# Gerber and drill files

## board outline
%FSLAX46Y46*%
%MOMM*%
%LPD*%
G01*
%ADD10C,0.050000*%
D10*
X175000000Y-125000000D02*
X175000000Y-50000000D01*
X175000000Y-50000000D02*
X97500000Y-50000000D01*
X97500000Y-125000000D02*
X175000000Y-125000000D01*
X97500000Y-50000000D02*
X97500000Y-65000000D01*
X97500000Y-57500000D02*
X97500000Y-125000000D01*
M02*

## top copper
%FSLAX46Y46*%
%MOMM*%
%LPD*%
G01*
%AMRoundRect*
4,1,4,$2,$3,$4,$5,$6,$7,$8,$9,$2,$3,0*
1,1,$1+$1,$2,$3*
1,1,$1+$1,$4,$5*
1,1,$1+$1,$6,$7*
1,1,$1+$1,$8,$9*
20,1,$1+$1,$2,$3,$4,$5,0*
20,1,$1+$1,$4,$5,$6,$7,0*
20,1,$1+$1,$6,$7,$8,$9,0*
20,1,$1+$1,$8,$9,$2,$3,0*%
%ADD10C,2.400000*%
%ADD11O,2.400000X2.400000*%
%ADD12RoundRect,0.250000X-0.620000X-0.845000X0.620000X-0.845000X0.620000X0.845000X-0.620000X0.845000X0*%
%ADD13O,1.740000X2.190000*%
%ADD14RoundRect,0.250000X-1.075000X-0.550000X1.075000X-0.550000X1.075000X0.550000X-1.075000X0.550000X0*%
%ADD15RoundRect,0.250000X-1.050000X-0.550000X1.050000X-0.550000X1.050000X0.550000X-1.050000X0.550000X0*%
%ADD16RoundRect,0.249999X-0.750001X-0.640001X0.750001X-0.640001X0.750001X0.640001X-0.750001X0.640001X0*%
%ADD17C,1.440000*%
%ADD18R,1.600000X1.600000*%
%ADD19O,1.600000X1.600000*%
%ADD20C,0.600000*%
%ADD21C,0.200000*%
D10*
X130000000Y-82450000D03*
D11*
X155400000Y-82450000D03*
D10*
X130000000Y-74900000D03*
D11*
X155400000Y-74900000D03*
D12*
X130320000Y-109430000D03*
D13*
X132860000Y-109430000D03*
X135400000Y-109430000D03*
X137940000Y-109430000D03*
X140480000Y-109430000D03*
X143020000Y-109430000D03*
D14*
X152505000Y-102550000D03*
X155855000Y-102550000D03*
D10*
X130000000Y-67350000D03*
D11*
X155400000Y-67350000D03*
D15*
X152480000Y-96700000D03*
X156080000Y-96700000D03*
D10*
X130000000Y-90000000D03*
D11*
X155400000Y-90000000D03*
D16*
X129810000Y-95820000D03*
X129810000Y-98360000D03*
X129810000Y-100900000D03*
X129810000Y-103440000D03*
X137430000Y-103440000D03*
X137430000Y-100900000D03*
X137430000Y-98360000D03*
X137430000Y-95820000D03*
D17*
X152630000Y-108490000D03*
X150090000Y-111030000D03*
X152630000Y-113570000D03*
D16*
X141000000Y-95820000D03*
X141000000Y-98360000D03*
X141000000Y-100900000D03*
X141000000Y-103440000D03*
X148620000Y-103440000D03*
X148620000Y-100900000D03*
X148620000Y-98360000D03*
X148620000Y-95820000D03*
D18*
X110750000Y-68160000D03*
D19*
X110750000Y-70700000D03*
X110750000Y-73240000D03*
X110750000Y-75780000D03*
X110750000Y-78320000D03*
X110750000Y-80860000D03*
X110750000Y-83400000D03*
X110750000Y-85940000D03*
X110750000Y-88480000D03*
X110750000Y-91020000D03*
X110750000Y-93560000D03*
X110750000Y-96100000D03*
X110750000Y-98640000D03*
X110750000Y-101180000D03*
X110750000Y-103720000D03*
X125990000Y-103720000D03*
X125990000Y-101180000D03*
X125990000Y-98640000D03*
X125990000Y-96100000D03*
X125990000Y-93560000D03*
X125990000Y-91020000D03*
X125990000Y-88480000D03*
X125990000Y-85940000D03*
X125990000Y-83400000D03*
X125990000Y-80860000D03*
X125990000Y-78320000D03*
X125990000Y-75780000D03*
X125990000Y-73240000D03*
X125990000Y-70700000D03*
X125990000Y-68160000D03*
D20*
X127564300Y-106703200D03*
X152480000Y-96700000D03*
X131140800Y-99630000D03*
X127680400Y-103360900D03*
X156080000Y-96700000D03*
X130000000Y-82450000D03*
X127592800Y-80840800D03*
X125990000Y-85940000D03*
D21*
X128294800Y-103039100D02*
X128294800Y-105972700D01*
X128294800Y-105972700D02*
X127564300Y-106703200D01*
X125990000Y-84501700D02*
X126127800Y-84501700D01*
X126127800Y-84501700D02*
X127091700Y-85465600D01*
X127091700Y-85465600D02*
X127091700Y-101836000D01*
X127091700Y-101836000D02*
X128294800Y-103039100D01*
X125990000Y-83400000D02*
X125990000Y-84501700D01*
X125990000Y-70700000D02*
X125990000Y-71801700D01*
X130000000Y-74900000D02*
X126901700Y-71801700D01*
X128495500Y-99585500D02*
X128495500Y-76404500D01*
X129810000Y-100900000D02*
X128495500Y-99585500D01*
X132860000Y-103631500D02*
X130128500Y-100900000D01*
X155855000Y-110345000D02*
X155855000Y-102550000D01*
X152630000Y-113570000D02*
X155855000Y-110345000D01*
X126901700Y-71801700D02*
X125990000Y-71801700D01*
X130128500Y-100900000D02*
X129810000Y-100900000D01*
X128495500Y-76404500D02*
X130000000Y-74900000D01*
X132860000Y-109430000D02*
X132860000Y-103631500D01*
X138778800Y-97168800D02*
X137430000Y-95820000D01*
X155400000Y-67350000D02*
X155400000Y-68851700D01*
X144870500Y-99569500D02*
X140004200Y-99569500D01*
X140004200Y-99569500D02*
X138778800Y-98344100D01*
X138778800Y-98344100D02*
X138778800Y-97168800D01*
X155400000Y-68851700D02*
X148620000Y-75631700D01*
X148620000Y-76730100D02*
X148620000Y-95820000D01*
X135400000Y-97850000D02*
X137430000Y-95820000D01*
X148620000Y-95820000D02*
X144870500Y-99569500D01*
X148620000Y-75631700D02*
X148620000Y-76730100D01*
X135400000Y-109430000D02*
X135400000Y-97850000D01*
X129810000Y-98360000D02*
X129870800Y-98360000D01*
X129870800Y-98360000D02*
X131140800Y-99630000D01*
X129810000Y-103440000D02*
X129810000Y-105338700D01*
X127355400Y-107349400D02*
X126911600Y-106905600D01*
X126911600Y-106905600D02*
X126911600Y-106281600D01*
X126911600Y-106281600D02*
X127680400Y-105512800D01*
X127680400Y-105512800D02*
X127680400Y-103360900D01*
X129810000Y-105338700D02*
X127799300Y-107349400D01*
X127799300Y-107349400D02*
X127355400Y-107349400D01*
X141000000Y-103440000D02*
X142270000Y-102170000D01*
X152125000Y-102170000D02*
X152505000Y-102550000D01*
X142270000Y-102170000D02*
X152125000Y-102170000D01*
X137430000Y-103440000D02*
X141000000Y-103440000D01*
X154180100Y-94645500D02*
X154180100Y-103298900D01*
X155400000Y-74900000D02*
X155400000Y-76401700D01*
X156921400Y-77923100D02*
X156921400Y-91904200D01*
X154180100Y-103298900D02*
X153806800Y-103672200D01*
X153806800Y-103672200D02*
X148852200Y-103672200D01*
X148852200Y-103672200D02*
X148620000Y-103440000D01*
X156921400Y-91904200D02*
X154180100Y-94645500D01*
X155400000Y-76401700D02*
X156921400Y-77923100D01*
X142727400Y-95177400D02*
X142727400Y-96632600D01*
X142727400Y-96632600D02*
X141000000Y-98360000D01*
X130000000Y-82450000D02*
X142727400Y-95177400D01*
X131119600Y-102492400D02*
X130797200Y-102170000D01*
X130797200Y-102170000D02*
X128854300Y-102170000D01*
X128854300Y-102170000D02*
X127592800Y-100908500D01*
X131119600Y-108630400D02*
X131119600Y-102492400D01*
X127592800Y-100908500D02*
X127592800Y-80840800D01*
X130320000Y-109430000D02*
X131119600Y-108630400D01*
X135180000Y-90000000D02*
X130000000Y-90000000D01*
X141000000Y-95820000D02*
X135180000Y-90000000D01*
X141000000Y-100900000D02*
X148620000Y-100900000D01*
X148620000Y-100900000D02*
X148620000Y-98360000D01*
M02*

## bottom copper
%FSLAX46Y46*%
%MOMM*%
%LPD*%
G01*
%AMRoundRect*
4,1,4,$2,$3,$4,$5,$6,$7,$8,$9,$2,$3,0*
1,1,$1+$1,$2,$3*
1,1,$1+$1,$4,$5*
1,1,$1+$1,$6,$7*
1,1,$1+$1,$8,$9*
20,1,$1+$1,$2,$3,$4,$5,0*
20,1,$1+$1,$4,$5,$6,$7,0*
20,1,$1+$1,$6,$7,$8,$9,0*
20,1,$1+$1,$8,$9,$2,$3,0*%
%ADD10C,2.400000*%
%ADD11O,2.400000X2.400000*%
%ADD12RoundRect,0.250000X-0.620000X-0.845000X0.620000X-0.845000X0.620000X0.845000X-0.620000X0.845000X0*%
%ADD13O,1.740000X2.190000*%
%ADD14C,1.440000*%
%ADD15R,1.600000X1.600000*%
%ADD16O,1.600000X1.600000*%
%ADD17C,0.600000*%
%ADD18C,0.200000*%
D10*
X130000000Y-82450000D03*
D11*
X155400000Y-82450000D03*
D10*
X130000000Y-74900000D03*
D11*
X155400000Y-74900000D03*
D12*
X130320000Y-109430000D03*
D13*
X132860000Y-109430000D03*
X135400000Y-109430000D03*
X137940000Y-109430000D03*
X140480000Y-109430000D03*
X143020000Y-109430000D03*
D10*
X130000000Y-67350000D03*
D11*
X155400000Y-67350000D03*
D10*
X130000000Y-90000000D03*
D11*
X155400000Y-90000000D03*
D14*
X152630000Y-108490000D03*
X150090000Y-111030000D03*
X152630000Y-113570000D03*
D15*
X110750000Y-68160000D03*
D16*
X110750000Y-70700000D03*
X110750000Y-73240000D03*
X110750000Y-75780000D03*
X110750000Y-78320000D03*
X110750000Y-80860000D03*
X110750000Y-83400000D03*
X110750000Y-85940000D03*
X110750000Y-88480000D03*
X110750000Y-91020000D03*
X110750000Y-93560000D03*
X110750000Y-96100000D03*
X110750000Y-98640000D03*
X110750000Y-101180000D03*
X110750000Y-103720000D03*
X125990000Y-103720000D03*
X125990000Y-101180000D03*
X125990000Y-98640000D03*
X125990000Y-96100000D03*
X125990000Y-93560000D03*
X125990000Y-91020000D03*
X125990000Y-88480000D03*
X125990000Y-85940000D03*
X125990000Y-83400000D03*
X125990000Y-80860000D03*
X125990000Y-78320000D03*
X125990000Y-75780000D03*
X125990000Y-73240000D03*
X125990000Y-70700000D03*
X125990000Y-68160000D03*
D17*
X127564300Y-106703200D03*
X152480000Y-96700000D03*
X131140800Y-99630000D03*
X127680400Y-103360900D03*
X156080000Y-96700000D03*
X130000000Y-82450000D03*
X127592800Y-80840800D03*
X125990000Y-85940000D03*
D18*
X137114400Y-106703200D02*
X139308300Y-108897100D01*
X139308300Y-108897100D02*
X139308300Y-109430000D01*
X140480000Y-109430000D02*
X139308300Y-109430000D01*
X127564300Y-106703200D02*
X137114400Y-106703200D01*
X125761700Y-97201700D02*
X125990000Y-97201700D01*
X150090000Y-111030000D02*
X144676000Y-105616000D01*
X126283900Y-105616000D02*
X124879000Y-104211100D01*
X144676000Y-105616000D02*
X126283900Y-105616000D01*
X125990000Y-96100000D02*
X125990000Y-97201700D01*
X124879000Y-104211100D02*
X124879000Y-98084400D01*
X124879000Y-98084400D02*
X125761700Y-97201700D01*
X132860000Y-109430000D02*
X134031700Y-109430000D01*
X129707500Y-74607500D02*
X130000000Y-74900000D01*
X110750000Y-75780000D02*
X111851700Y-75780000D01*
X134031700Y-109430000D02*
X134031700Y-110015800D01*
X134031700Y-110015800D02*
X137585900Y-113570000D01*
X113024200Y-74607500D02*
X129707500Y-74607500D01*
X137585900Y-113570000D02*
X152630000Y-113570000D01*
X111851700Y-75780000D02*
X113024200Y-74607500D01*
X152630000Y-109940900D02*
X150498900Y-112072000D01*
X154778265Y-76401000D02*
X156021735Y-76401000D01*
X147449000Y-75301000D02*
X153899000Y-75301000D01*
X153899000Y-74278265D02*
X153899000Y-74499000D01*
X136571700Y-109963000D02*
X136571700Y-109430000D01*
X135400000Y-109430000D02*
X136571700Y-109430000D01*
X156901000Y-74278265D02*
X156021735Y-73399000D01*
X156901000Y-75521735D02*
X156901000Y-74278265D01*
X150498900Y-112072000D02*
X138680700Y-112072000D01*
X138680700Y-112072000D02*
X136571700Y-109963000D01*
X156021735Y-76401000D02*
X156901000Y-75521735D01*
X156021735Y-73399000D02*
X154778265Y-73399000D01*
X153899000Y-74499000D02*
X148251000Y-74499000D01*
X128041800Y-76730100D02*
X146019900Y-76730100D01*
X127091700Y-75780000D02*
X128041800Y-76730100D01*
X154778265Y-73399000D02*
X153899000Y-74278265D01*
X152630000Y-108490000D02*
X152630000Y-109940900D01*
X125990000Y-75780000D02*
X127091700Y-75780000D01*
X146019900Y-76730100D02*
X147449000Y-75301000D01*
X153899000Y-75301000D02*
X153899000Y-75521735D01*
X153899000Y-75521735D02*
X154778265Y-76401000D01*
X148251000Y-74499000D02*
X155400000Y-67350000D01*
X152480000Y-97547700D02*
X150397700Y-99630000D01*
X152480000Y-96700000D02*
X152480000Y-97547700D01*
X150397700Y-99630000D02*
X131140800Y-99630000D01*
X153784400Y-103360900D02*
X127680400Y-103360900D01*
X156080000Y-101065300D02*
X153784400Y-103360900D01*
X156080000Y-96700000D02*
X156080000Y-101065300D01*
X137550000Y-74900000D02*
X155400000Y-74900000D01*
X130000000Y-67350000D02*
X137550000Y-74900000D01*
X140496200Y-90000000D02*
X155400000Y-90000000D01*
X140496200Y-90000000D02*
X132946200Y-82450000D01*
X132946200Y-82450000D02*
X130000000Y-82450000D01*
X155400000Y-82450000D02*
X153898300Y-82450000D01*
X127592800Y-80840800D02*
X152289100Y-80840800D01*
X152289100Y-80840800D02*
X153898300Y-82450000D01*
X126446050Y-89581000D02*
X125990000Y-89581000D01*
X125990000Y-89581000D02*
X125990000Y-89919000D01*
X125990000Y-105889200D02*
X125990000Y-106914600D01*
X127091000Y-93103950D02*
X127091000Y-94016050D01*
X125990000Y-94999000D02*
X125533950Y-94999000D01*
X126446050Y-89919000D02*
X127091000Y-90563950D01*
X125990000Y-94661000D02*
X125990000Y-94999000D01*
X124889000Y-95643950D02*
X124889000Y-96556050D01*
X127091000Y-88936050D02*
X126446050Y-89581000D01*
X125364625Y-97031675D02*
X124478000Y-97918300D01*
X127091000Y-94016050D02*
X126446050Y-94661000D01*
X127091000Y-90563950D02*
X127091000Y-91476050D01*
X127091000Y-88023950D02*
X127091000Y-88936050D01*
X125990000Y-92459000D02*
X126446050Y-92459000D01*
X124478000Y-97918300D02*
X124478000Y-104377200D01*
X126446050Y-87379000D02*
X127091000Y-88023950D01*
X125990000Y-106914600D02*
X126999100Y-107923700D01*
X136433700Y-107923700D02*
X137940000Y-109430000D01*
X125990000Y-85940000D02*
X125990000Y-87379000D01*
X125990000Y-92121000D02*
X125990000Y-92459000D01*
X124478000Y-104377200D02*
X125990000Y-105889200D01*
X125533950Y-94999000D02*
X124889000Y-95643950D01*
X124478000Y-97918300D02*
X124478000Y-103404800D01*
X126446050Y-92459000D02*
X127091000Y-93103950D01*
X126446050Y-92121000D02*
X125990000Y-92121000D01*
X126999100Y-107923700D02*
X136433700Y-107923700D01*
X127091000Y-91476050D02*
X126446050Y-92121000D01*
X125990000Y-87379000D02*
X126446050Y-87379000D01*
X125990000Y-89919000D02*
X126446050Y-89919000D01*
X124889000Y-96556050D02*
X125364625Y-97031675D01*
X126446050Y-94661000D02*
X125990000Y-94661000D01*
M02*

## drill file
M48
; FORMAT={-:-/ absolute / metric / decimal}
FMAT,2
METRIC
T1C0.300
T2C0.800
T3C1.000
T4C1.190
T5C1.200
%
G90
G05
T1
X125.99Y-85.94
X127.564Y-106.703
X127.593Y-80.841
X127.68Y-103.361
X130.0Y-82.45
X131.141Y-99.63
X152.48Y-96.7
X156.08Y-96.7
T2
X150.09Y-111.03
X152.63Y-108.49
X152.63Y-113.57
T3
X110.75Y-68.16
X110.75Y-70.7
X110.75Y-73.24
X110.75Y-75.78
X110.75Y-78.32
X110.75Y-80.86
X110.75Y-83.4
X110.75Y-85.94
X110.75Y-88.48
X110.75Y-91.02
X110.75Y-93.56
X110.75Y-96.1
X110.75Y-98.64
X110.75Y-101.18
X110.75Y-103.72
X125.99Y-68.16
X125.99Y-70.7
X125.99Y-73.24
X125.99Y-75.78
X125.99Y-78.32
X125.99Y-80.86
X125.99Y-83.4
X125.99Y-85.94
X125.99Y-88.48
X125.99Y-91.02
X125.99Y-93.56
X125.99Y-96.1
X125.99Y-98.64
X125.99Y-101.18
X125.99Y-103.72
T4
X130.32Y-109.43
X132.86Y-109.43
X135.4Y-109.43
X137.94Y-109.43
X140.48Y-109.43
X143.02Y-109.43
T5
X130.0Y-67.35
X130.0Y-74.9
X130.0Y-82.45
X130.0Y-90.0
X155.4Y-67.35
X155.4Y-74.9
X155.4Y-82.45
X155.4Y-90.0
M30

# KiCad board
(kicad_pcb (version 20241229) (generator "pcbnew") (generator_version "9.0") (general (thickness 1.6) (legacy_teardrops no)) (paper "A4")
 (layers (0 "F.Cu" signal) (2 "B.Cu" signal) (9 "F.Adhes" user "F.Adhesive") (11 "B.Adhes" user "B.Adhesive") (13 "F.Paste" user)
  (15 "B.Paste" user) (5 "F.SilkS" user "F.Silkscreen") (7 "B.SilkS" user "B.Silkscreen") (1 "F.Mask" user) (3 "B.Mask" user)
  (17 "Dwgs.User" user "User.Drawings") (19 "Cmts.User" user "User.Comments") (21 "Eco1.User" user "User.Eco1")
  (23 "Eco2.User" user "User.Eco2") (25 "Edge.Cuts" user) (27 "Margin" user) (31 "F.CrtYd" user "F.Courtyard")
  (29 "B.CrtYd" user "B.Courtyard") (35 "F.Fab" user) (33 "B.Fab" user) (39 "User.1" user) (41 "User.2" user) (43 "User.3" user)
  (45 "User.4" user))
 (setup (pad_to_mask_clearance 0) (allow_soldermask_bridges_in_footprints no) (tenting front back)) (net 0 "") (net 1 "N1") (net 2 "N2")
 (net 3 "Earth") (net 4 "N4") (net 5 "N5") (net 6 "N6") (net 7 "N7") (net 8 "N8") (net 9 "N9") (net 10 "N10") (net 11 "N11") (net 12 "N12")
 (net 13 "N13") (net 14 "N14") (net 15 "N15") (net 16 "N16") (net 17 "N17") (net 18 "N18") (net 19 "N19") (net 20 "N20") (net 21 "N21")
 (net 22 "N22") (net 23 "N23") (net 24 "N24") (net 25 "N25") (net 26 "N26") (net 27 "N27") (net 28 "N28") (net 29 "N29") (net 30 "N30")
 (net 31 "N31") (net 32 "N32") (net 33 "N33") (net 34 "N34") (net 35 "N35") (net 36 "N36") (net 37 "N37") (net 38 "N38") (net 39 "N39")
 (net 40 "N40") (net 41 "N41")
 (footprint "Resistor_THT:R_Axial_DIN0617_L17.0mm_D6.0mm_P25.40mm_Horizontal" (layer "F.Cu") (at 130 82.45)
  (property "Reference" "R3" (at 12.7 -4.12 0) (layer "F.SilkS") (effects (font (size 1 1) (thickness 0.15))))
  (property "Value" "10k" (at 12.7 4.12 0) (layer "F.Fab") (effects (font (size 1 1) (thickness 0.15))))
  (pad "1" thru_hole circle (at 0 0) (size 2.4 2.4) (drill 1.2) (layers "*.Cu" "*.Mask") (remove_unused_layers no) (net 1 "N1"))
  (pad "2" thru_hole oval (at 25.4 0) (size 2.4 2.4) (drill 1.2) (layers "*.Cu" "*.Mask") (remove_unused_layers no) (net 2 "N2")))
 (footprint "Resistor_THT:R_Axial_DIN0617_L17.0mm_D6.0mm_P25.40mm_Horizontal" (layer "F.Cu") (at 130 74.9)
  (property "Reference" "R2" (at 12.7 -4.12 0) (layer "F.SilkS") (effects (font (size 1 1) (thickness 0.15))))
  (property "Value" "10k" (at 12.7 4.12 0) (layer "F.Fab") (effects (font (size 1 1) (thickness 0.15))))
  (pad "1" thru_hole circle (at 0 0) (size 2.4 2.4) (drill 1.2) (layers "*.Cu" "*.Mask") (remove_unused_layers no) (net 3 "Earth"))
  (pad "2" thru_hole oval (at 25.4 0) (size 2.4 2.4) (drill 1.2) (layers "*.Cu" "*.Mask") (remove_unused_layers no) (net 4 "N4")))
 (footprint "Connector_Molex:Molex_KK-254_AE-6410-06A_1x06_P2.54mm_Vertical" (layer "F.Cu") (at 130.32 109.43)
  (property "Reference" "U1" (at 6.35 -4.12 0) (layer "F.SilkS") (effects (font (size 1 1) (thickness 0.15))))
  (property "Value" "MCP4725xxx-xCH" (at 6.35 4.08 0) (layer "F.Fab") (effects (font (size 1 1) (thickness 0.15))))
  (pad "1" thru_hole roundrect (at 0 0) (size 1.74 2.19) (drill 1.19) (layers "*.Cu" "*.Mask") (remove_unused_layers no)
   (roundrect_rratio 0.143678) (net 2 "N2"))
  (pad "2" thru_hole oval (at 2.54 0) (size 1.74 2.19) (drill 1.19) (layers "*.Cu" "*.Mask") (remove_unused_layers no) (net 3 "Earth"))
  (pad "3" thru_hole oval (at 5.08 0) (size 1.74 2.19) (drill 1.19) (layers "*.Cu" "*.Mask") (remove_unused_layers no) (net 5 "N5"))
  (pad "4" thru_hole oval (at 7.62 0) (size 1.74 2.19) (drill 1.19) (layers "*.Cu" "*.Mask") (remove_unused_layers no) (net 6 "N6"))
  (pad "5" thru_hole oval (at 10.16 0) (size 1.74 2.19) (drill 1.19) (layers "*.Cu" "*.Mask") (remove_unused_layers no) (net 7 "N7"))
  (pad "6" thru_hole oval (at 12.7 0) (size 1.74 2.19) (drill 1.19) (layers "*.Cu" "*.Mask") (remove_unused_layers no) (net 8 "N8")))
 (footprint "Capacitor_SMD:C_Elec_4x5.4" (layer "F.Cu") (at 154.18 102.55)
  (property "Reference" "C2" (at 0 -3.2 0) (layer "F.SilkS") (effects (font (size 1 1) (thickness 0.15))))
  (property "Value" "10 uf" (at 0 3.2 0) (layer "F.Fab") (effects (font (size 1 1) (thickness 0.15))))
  (pad "1" smd roundrect (at -1.675 0) (size 2.65 1.6) (layers "F.Cu" "F.Mask" "F.Paste") (roundrect_rratio 0.15625) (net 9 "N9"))
  (pad "2" smd roundrect (at 1.675 0) (size 2.65 1.6) (layers "F.Cu" "F.Mask" "F.Paste") (roundrect_rratio 0.15625) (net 3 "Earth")))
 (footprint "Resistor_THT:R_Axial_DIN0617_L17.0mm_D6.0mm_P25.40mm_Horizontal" (layer "F.Cu") (at 130 67.35)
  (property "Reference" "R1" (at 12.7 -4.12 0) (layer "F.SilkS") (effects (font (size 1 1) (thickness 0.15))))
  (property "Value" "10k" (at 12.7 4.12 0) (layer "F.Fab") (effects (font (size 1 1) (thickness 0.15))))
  (pad "1" thru_hole circle (at 0 0) (size 2.4 2.4) (drill 1.2) (layers "*.Cu" "*.Mask") (remove_unused_layers no) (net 4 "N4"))
  (pad "2" thru_hole oval (at 25.4 0) (size 2.4 2.4) (drill 1.2) (layers "*.Cu" "*.Mask") (remove_unused_layers no) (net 5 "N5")))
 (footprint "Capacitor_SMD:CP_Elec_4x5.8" (layer "F.Cu") (at 154.28 96.7)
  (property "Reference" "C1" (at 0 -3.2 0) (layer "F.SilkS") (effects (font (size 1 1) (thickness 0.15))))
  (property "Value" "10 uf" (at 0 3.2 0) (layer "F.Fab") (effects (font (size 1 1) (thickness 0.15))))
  (pad "1" smd roundrect (at -1.8 0) (size 2.6 1.6) (layers "F.Cu" "F.Mask" "F.Paste") (roundrect_rratio 0.15625) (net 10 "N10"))
  (pad "2" smd roundrect (at 1.8 0) (size 2.6 1.6) (layers "F.Cu" "F.Mask" "F.Paste") (roundrect_rratio 0.15625) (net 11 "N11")))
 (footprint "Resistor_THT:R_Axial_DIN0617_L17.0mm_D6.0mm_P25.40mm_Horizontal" (layer "F.Cu") (at 130 90)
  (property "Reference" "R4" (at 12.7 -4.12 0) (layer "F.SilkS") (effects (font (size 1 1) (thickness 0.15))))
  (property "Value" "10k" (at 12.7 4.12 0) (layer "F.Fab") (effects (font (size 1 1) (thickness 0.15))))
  (pad "1" thru_hole circle (at 0 0) (size 2.4 2.4) (drill 1.2) (layers "*.Cu" "*.Mask") (remove_unused_layers no) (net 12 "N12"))
  (pad "2" thru_hole oval (at 25.4 0) (size 2.4 2.4) (drill 1.2) (layers "*.Cu" "*.Mask") (remove_unused_layers no) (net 1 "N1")))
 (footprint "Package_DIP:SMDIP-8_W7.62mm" (layer "F.Cu") (at 133.62 99.63)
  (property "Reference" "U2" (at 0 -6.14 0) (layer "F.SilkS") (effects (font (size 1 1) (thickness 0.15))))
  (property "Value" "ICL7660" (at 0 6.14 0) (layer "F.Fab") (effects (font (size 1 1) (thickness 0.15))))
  (pad "1" smd roundrect (at -3.81 -3.81) (size 2 1.78) (layers "F.Cu" "F.Mask" "F.Paste") (roundrect_rratio 0.140449) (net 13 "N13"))
  (pad "2" smd roundrect (at -3.81 -1.27) (size 2 1.78) (layers "F.Cu" "F.Mask" "F.Paste") (roundrect_rratio 0.140449) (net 10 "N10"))
  (pad "3" smd roundrect (at -3.81 1.27) (size 2 1.78) (layers "F.Cu" "F.Mask" "F.Paste") (roundrect_rratio 0.140449) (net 3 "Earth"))
  (pad "4" smd roundrect (at -3.81 3.81) (size 2 1.78) (layers "F.Cu" "F.Mask" "F.Paste") (roundrect_rratio 0.140449) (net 11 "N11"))
  (pad "5" smd roundrect (at 3.81 3.81) (size 2 1.78) (layers "F.Cu" "F.Mask" "F.Paste") (roundrect_rratio 0.140449) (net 9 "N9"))
  (pad "6" smd roundrect (at 3.81 1.27) (size 2 1.78) (layers "F.Cu" "F.Mask" "F.Paste") (roundrect_rratio 0.140449) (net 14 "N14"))
  (pad "7" smd roundrect (at 3.81 -1.27) (size 2 1.78) (layers "F.Cu" "F.Mask" "F.Paste") (roundrect_rratio 0.140449) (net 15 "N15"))
  (pad "8" smd roundrect (at 3.81 -3.81) (size 2 1.78) (layers "F.Cu" "F.Mask" "F.Paste") (roundrect_rratio 0.140449) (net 5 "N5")))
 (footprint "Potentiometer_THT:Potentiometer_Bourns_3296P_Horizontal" (layer "F.Cu") (at 152.63 108.49)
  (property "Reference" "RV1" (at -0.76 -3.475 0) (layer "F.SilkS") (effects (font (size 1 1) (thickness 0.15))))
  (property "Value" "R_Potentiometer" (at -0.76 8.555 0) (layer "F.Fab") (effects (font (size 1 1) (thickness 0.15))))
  (pad "1" thru_hole circle (at 0 0) (size 1.44 1.44) (drill 0.8) (layers "*.Cu" "*.Mask") (remove_unused_layers no) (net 5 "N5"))
  (pad "2" thru_hole circle (at -2.54 2.54) (size 1.44 1.44) (drill 0.8) (layers "*.Cu" "*.Mask") (remove_unused_layers no) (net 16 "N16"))
  (pad "3" thru_hole circle (at 0 5.08) (size 1.44 1.44) (drill 0.8) (layers "*.Cu" "*.Mask") (remove_unused_layers no) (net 3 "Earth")))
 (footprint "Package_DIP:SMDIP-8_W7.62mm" (layer "F.Cu") (at 144.81 99.63)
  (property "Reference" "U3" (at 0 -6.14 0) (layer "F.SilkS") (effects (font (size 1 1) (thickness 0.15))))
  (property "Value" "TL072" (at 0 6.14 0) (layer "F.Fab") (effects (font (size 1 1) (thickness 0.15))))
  (pad "1" smd roundrect (at -3.81 -3.81) (size 2 1.78) (layers "F.Cu" "F.Mask" "F.Paste") (roundrect_rratio 0.140449) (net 12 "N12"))
  (pad "2" smd roundrect (at -3.81 -1.27) (size 2 1.78) (layers "F.Cu" "F.Mask" "F.Paste") (roundrect_rratio 0.140449) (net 1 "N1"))
  (pad "3" smd roundrect (at -3.81 1.27) (size 2 1.78) (layers "F.Cu" "F.Mask" "F.Paste") (roundrect_rratio 0.140449) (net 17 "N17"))
  (pad "4" smd roundrect (at -3.81 3.81) (size 2 1.78) (layers "F.Cu" "F.Mask" "F.Paste") (roundrect_rratio 0.140449) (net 9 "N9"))
  (pad "5" smd roundrect (at 3.81 3.81) (size 2 1.78) (layers "F.Cu" "F.Mask" "F.Paste") (roundrect_rratio 0.140449) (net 4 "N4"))
  (pad "6" smd roundrect (at 3.81 1.27) (size 2 1.78) (layers "F.Cu" "F.Mask" "F.Paste") (roundrect_rratio 0.140449) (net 17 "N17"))
  (pad "7" smd roundrect (at 3.81 -1.27) (size 2 1.78) (layers "F.Cu" "F.Mask" "F.Paste") (roundrect_rratio 0.140449) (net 17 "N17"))
  (pad "8" smd roundrect (at 3.81 -3.81) (size 2 1.78) (layers "F.Cu" "F.Mask" "F.Paste") (roundrect_rratio 0.140449) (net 5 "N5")))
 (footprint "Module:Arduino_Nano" (layer "F.Cu") (at 110.75 68.16)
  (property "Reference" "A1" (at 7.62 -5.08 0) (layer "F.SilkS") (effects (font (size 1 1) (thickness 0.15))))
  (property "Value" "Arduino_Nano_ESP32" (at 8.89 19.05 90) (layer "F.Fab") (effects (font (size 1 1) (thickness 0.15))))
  (pad "1" thru_hole rect (at 0 0) (size 1.6 1.6) (drill 1) (layers "*.Cu" "*.Mask") (remove_unused_layers no) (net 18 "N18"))
  (pad "2" thru_hole oval (at 0 2.54) (size 1.6 1.6) (drill 1) (layers "*.Cu" "*.Mask") (remove_unused_layers no) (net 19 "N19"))
  (pad "3" thru_hole oval (at 0 5.08) (size 1.6 1.6) (drill 1) (layers "*.Cu" "*.Mask") (remove_unused_layers no) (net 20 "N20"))
  (pad "4" thru_hole oval (at 0 7.62) (size 1.6 1.6) (drill 1) (layers "*.Cu" "*.Mask") (remove_unused_layers no) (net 3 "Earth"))
  (pad "5" thru_hole oval (at 0 10.16) (size 1.6 1.6) (drill 1) (layers "*.Cu" "*.Mask") (remove_unused_layers no) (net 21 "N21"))
  (pad "6" thru_hole oval (at 0 12.7) (size 1.6 1.6) (drill 1) (layers "*.Cu" "*.Mask") (remove_unused_layers no) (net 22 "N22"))
  (pad "7" thru_hole oval (at 0 15.24) (size 1.6 1.6) (drill 1) (layers "*.Cu" "*.Mask") (remove_unused_layers no) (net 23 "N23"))
  (pad "8" thru_hole oval (at 0 17.78) (size 1.6 1.6) (drill 1) (layers "*.Cu" "*.Mask") (remove_unused_layers no) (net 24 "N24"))
  (pad "9" thru_hole oval (at 0 20.32) (size 1.6 1.6) (drill 1) (layers "*.Cu" "*.Mask") (remove_unused_layers no) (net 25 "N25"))
  (pad "10" thru_hole oval (at 0 22.86) (size 1.6 1.6) (drill 1) (layers "*.Cu" "*.Mask") (remove_unused_layers no) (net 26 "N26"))
  (pad "11" thru_hole oval (at 0 25.4) (size 1.6 1.6) (drill 1) (layers "*.Cu" "*.Mask") (remove_unused_layers no) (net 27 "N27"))
  (pad "12" thru_hole oval (at 0 27.94) (size 1.6 1.6) (drill 1) (layers "*.Cu" "*.Mask") (remove_unused_layers no) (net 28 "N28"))
  (pad "13" thru_hole oval (at 0 30.48) (size 1.6 1.6) (drill 1) (layers "*.Cu" "*.Mask") (remove_unused_layers no) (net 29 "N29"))
  (pad "14" thru_hole oval (at 0 33.02) (size 1.6 1.6) (drill 1) (layers "*.Cu" "*.Mask") (remove_unused_layers no) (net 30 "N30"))
  (pad "15" thru_hole oval (at 0 35.56) (size 1.6 1.6) (drill 1) (layers "*.Cu" "*.Mask") (remove_unused_layers no) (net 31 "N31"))
  (pad "16" thru_hole oval (at 15.24 35.56) (size 1.6 1.6) (drill 1) (layers "*.Cu" "*.Mask") (remove_unused_layers no) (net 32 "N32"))
  (pad "17" thru_hole oval (at 15.24 33.02) (size 1.6 1.6) (drill 1) (layers "*.Cu" "*.Mask") (remove_unused_layers no) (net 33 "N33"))
  (pad "18" thru_hole oval (at 15.24 30.48) (size 1.6 1.6) (drill 1) (layers "*.Cu" "*.Mask") (remove_unused_layers no) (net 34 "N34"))
  (pad "19" thru_hole oval (at 15.24 27.94) (size 1.6 1.6) (drill 1) (layers "*.Cu" "*.Mask") (remove_unused_layers no) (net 16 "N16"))
  (pad "20" thru_hole oval (at 15.24 25.4) (size 1.6 1.6) (drill 1) (layers "*.Cu" "*.Mask") (remove_unused_layers no) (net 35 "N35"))
  (pad "21" thru_hole oval (at 15.24 22.86) (size 1.6 1.6) (drill 1) (layers "*.Cu" "*.Mask") (remove_unused_layers no) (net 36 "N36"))
  (pad "22" thru_hole oval (at 15.24 20.32) (size 1.6 1.6) (drill 1) (layers "*.Cu" "*.Mask") (remove_unused_layers no) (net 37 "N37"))
  (pad "23" thru_hole oval (at 15.24 17.78) (size 1.6 1.6) (drill 1) (layers "*.Cu" "*.Mask") (remove_unused_layers no) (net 6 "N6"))
  (pad "24" thru_hole oval (at 15.24 15.24) (size 1.6 1.6) (drill 1) (layers "*.Cu" "*.Mask") (remove_unused_layers no) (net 7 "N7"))
  (pad "25" thru_hole oval (at 15.24 12.7) (size 1.6 1.6) (drill 1) (layers "*.Cu" "*.Mask") (remove_unused_layers no) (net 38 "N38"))
  (pad "26" thru_hole oval (at 15.24 10.16) (size 1.6 1.6) (drill 1) (layers "*.Cu" "*.Mask") (remove_unused_layers no) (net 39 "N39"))
  (pad "27" thru_hole oval (at 15.24 7.62) (size 1.6 1.6) (drill 1) (layers "*.Cu" "*.Mask") (remove_unused_layers no) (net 5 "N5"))
  (pad "28" thru_hole oval (at 15.24 5.08) (size 1.6 1.6) (drill 1) (layers "*.Cu" "*.Mask") (remove_unused_layers no) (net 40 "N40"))
  (pad "29" thru_hole oval (at 15.24 2.54) (size 1.6 1.6) (drill 1) (layers "*.Cu" "*.Mask") (remove_unused_layers no) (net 3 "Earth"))
  (pad "30" thru_hole oval (at 15.24 0) (size 1.6 1.6) (drill 1) (layers "*.Cu" "*.Mask") (remove_unused_layers no) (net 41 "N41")))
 (gr_line (start 175 125) (end 175 50) (stroke (width 0.05) (type default)) (layer "Edge.Cuts"))
 (gr_line (start 175 50) (end 97.5 50) (stroke (width 0.05) (type default)) (layer "Edge.Cuts"))
 (gr_line (start 97.5 125) (end 175 125) (stroke (width 0.05) (type default)) (layer "Edge.Cuts"))
 (gr_line (start 97.5 50) (end 97.5 65) (stroke (width 0.05) (type default)) (layer "Edge.Cuts"))
 (gr_line (start 97.5 57.5) (end 97.5 125) (stroke (width 0.05) (type default)) (layer "Edge.Cuts"))
 (segment (start 128.2948 103.0391) (end 128.2948 105.9727) (width 0.2) (layer "F.Cu") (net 7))
 (segment (start 128.2948 105.9727) (end 127.5643 106.7032) (width 0.2) (layer "F.Cu") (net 7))
 (segment (start 125.99 84.5017) (end 126.1278 84.5017) (width 0.2) (layer "F.Cu") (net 7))
 (segment (start 126.1278 84.5017) (end 127.0917 85.4656) (width 0.2) (layer "F.Cu") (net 7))
 (segment (start 127.0917 85.4656) (end 127.0917 101.836) (width 0.2) (layer "F.Cu") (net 7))
 (segment (start 127.0917 101.836) (end 128.2948 103.0391) (width 0.2) (layer "F.Cu") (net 7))
 (segment (start 125.99 83.4) (end 125.99 84.5017) (width 0.2) (layer "F.Cu") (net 7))
 (via (at 127.5643 106.7032) (size 0.6) (drill 0.3) (layers "F.Cu" "B.Cu") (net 7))
 (segment (start 137.1144 106.7032) (end 139.3083 108.8971) (width 0.2) (layer "B.Cu") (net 7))
 (segment (start 139.3083 108.8971) (end 139.3083 109.43) (width 0.2) (layer "B.Cu") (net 7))
 (segment (start 140.48 109.43) (end 139.3083 109.43) (width 0.2) (layer "B.Cu") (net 7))
 (segment (start 127.5643 106.7032) (end 137.1144 106.7032) (width 0.2) (layer "B.Cu") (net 7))
 (segment (start 125.7617 97.2017) (end 125.99 97.2017) (width 0.2) (layer "B.Cu") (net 16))
 (segment (start 150.09 111.03) (end 144.676 105.616) (width 0.2) (layer "B.Cu") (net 16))
 (segment (start 126.2839 105.616) (end 124.879 104.2111) (width 0.2) (layer "B.Cu") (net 16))
 (segment (start 144.676 105.616) (end 126.2839 105.616) (width 0.2) (layer "B.Cu") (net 16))
 (segment (start 125.99 96.1) (end 125.99 97.2017) (width 0.2) (layer "B.Cu") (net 16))
 (segment (start 124.879 104.2111) (end 124.879 98.0844) (width 0.2) (layer "B.Cu") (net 16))
 (segment (start 124.879 98.0844) (end 125.7617 97.2017) (width 0.2) (layer "B.Cu") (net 16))
 (segment (start 125.99 70.7) (end 125.99 71.8017) (width 0.2) (layer "F.Cu") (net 3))
 (segment (start 130 74.9) (end 126.9017 71.8017) (width 0.2) (layer "F.Cu") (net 3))
 (segment (start 128.4955 99.5855) (end 128.4955 76.4045) (width 0.2) (layer "F.Cu") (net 3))
 (segment (start 129.81 100.9) (end 128.4955 99.5855) (width 0.2) (layer "F.Cu") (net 3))
 (segment (start 132.86 103.6315) (end 130.1285 100.9) (width 0.2) (layer "F.Cu") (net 3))
 (segment (start 155.855 110.345) (end 155.855 102.55) (width 0.2) (layer "F.Cu") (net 3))
 (segment (start 152.63 113.57) (end 155.855 110.345) (width 0.2) (layer "F.Cu") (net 3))
 (segment (start 126.9017 71.8017) (end 125.99 71.8017) (width 0.2) (layer "F.Cu") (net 3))
 (segment (start 130.1285 100.9) (end 129.81 100.9) (width 0.2) (layer "F.Cu") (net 3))
 (segment (start 128.4955 76.4045) (end 130 74.9) (width 0.2) (layer "F.Cu") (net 3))
 (segment (start 132.86 109.43) (end 132.86 103.6315) (width 0.2) (layer "F.Cu") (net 3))
 (segment (start 132.86 109.43) (end 134.0317 109.43) (width 0.2) (layer "B.Cu") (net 3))
 (segment (start 129.7075 74.6075) (end 130 74.9) (width 0.2) (layer "B.Cu") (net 3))
 (segment (start 110.75 75.78) (end 111.8517 75.78) (width 0.2) (layer "B.Cu") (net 3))
 (segment (start 134.0317 109.43) (end 134.0317 110.0158) (width 0.2) (layer "B.Cu") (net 3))
 (segment (start 134.0317 110.0158) (end 137.5859 113.57) (width 0.2) (layer "B.Cu") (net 3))
 (segment (start 113.0242 74.6075) (end 129.7075 74.6075) (width 0.2) (layer "B.Cu") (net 3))
 (segment (start 137.5859 113.57) (end 152.63 113.57) (width 0.2) (layer "B.Cu") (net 3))
 (segment (start 111.8517 75.78) (end 113.0242 74.6075) (width 0.2) (layer "B.Cu") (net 3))
 (segment (start 138.7788 97.1688) (end 137.43 95.82) (width 0.2) (layer "F.Cu") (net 5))
 (segment (start 155.4 67.35) (end 155.4 68.8517) (width 0.2) (layer "F.Cu") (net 5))
 (segment (start 144.8705 99.5695) (end 140.0042 99.5695) (width 0.2) (layer "F.Cu") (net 5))
 (segment (start 140.0042 99.5695) (end 138.7788 98.3441) (width 0.2) (layer "F.Cu") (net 5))
 (segment (start 138.7788 98.3441) (end 138.7788 97.1688) (width 0.2) (layer "F.Cu") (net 5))
 (segment (start 155.4 68.8517) (end 148.62 75.6317) (width 0.2) (layer "F.Cu") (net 5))
 (segment (start 148.62 76.7301) (end 148.62 95.82) (width 0.2) (layer "F.Cu") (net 5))
 (segment (start 135.4 97.85) (end 137.43 95.82) (width 0.2) (layer "F.Cu") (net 5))
 (segment (start 148.62 95.82) (end 144.8705 99.5695) (width 0.2) (layer "F.Cu") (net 5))
 (segment (start 148.62 75.6317) (end 148.62 76.7301) (width 0.2) (layer "F.Cu") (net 5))
 (segment (start 135.4 109.43) (end 135.4 97.85) (width 0.2) (layer "F.Cu") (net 5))
 (segment (start 152.63 109.9409) (end 150.4989 112.072) (width 0.2) (layer "B.Cu") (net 5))
 (segment (start 154.778265 76.401) (end 156.021735 76.401) (width 0.2) (layer "B.Cu") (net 5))
 (segment (start 147.449 75.301) (end 153.899 75.301) (width 0.2) (layer "B.Cu") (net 5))
 (segment (start 153.899 74.278265) (end 153.899 74.499) (width 0.2) (layer "B.Cu") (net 5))
 (segment (start 136.5717 109.963) (end 136.5717 109.43) (width 0.2) (layer "B.Cu") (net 5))
 (segment (start 135.4 109.43) (end 136.5717 109.43) (width 0.2) (layer "B.Cu") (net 5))
 (segment (start 156.901 74.278265) (end 156.021735 73.399) (width 0.2) (layer "B.Cu") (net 5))
 (segment (start 156.901 75.521735) (end 156.901 74.278265) (width 0.2) (layer "B.Cu") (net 5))
 (segment (start 150.4989 112.072) (end 138.6807 112.072) (width 0.2) (layer "B.Cu") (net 5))
 (segment (start 138.6807 112.072) (end 136.5717 109.963) (width 0.2) (layer "B.Cu") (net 5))
 (segment (start 156.021735 76.401) (end 156.901 75.521735) (width 0.2) (layer "B.Cu") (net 5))
 (segment (start 156.021735 73.399) (end 154.778265 73.399) (width 0.2) (layer "B.Cu") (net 5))
 (segment (start 153.899 74.499) (end 148.251 74.499) (width 0.2) (layer "B.Cu") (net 5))
 (segment (start 128.0418 76.7301) (end 146.0199 76.7301) (width 0.2) (layer "B.Cu") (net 5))
 (segment (start 127.0917 75.78) (end 128.0418 76.7301) (width 0.2) (layer "B.Cu") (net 5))
 (segment (start 154.778265 73.399) (end 153.899 74.278265) (width 0.2) (layer "B.Cu") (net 5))
 (segment (start 152.63 108.49) (end 152.63 109.9409) (width 0.2) (layer "B.Cu") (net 5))
 (segment (start 125.99 75.78) (end 127.0917 75.78) (width 0.2) (layer "B.Cu") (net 5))
 (segment (start 146.0199 76.7301) (end 147.449 75.301) (width 0.2) (layer "B.Cu") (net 5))
 (segment (start 153.899 75.301) (end 153.899 75.521735) (width 0.2) (layer "B.Cu") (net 5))
 (segment (start 153.899 75.521735) (end 154.778265 76.401) (width 0.2) (layer "B.Cu") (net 5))
 (segment (start 148.251 74.499) (end 155.4 67.35) (width 0.2) (layer "B.Cu") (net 5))
 (segment (start 129.81 98.36) (end 129.8708 98.36) (width 0.2) (layer "F.Cu") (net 10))
 (segment (start 129.8708 98.36) (end 131.1408 99.63) (width 0.2) (layer "F.Cu") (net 10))
 (via (at 152.48 96.7) (size 0.6) (drill 0.3) (layers "F.Cu" "B.Cu") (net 10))
 (via (at 131.1408 99.63) (size 0.6) (drill 0.3) (layers "F.Cu" "B.Cu") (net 10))
 (segment (start 152.48 97.5477) (end 150.3977 99.63) (width 0.2) (layer "B.Cu") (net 10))
 (segment (start 152.48 96.7) (end 152.48 97.5477) (width 0.2) (layer "B.Cu") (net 10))
 (segment (start 150.3977 99.63) (end 131.1408 99.63) (width 0.2) (layer "B.Cu") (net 10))
 (segment (start 129.81 103.44) (end 129.81 105.3387) (width 0.2) (layer "F.Cu") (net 11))
 (segment (start 127.3554 107.3494) (end 126.9116 106.9056) (width 0.2) (layer "F.Cu") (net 11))
 (segment (start 126.9116 106.9056) (end 126.9116 106.2816) (width 0.2) (layer "F.Cu") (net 11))
 (segment (start 126.9116 106.2816) (end 127.6804 105.5128) (width 0.2) (layer "F.Cu") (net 11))
 (segment (start 127.6804 105.5128) (end 127.6804 103.3609) (width 0.2) (layer "F.Cu") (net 11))
 (segment (start 129.81 105.3387) (end 127.7993 107.3494) (width 0.2) (layer "F.Cu") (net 11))
 (segment (start 127.7993 107.3494) (end 127.3554 107.3494) (width 0.2) (layer "F.Cu") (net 11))
 (via (at 127.6804 103.3609) (size 0.6) (drill 0.3) (layers "F.Cu" "B.Cu") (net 11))
 (via (at 156.08 96.7) (size 0.6) (drill 0.3) (layers "F.Cu" "B.Cu") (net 11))
 (segment (start 153.7844 103.3609) (end 127.6804 103.3609) (width 0.2) (layer "B.Cu") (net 11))
 (segment (start 156.08 101.0653) (end 153.7844 103.3609) (width 0.2) (layer "B.Cu") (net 11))
 (segment (start 156.08 96.7) (end 156.08 101.0653) (width 0.2) (layer "B.Cu") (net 11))
 (segment (start 141 103.44) (end 142.27 102.17) (width 0.2) (layer "F.Cu") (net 9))
 (segment (start 152.125 102.17) (end 152.505 102.55) (width 0.2) (layer "F.Cu") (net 9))
 (segment (start 142.27 102.17) (end 152.125 102.17) (width 0.2) (layer "F.Cu") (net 9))
 (segment (start 137.43 103.44) (end 141 103.44) (width 0.2) (layer "F.Cu") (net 9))
 (segment (start 154.1801 94.6455) (end 154.1801 103.2989) (width 0.2) (layer "F.Cu") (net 4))
 (segment (start 155.4 74.9) (end 155.4 76.4017) (width 0.2) (layer "F.Cu") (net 4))
 (segment (start 156.9214 77.9231) (end 156.9214 91.9042) (width 0.2) (layer "F.Cu") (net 4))
 (segment (start 154.1801 103.2989) (end 153.8068 103.6722) (width 0.2) (layer "F.Cu") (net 4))
 (segment (start 153.8068 103.6722) (end 148.8522 103.6722) (width 0.2) (layer "F.Cu") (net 4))
 (segment (start 148.8522 103.6722) (end 148.62 103.44) (width 0.2) (layer "F.Cu") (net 4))
 (segment (start 156.9214 91.9042) (end 154.1801 94.6455) (width 0.2) (layer "F.Cu") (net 4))
 (segment (start 155.4 76.4017) (end 156.9214 77.9231) (width 0.2) (layer "F.Cu") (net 4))
 (segment (start 137.55 74.9) (end 155.4 74.9) (width 0.2) (layer "B.Cu") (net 4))
 (segment (start 130 67.35) (end 137.55 74.9) (width 0.2) (layer "B.Cu") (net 4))
 (segment (start 142.7274 95.1774) (end 142.7274 96.6326) (width 0.2) (layer "F.Cu") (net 1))
 (segment (start 142.7274 96.6326) (end 141 98.36) (width 0.2) (layer "F.Cu") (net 1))
 (segment (start 130 82.45) (end 142.7274 95.1774) (width 0.2) (layer "F.Cu") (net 1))
 (via (at 130 82.45) (size 0.6) (drill 0.3) (layers "F.Cu" "B.Cu") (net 1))
 (segment (start 140.4962 90) (end 155.4 90) (width 0.2) (layer "B.Cu") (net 1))
 (segment (start 140.4962 90) (end 132.9462 82.45) (width 0.2) (layer "B.Cu") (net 1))
 (segment (start 132.9462 82.45) (end 130 82.45) (width 0.2) (layer "B.Cu") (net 1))
 (segment (start 131.1196 102.4924) (end 130.7972 102.17) (width 0.2) (layer "F.Cu") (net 2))
 (segment (start 130.7972 102.17) (end 128.8543 102.17) (width 0.2) (layer "F.Cu") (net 2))
 (segment (start 128.8543 102.17) (end 127.5928 100.9085) (width 0.2) (layer "F.Cu") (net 2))
 (segment (start 131.1196 108.6304) (end 131.1196 102.4924) (width 0.2) (layer "F.Cu") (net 2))
 (segment (start 127.5928 100.9085) (end 127.5928 80.8408) (width 0.2) (layer "F.Cu") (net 2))
 (segment (start 130.32 109.43) (end 131.1196 108.6304) (width 0.2) (layer "F.Cu") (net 2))
 (via (at 127.5928 80.8408) (size 0.6) (drill 0.3) (layers "F.Cu" "B.Cu") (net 2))
 (segment (start 155.4 82.45) (end 153.8983 82.45) (width 0.2) (layer "B.Cu") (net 2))
 (segment (start 127.5928 80.8408) (end 152.2891 80.8408) (width 0.2) (layer "B.Cu") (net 2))
 (segment (start 152.2891 80.8408) (end 153.8983 82.45) (width 0.2) (layer "B.Cu") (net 2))
 (segment (start 135.18 90) (end 130 90) (width 0.2) (layer "F.Cu") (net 12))
 (segment (start 141 95.82) (end 135.18 90) (width 0.2) (layer "F.Cu") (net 12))
 (segment (start 141 100.9) (end 148.62 100.9) (width 0.2) (layer "F.Cu") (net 17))
 (segment (start 148.62 100.9) (end 148.62 98.36) (width 0.2) (layer "F.Cu") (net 17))
 (via (at 125.99 85.94) (size 0.6) (drill 0.3) (layers "F.Cu" "B.Cu") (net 6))
 (segment (start 126.44605 89.581) (end 125.99 89.581) (width 0.2) (layer "B.Cu") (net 6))
 (segment (start 125.99 89.581) (end 125.99 89.919) (width 0.2) (layer "B.Cu") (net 6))
 (segment (start 125.99 105.8892) (end 125.99 106.9146) (width 0.2) (layer "B.Cu") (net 6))
 (segment (start 127.091 93.10395) (end 127.091 94.01605) (width 0.2) (layer "B.Cu") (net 6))
 (segment (start 125.99 94.999) (end 125.53395 94.999) (width 0.2) (layer "B.Cu") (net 6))
 (segment (start 126.44605 89.919) (end 127.091 90.56395) (width 0.2) (layer "B.Cu") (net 6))
 (segment (start 125.99 94.661) (end 125.99 94.999) (width 0.2) (layer "B.Cu") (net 6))
 (segment (start 124.889 95.64395) (end 124.889 96.55605) (width 0.2) (layer "B.Cu") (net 6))
 (segment (start 127.091 88.93605) (end 126.44605 89.581) (width 0.2) (layer "B.Cu") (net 6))
 (segment (start 125.364625 97.031675) (end 124.478 97.9183) (width 0.2) (layer "B.Cu") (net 6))
 (segment (start 127.091 94.01605) (end 126.44605 94.661) (width 0.2) (layer "B.Cu") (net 6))
 (segment (start 127.091 90.56395) (end 127.091 91.47605) (width 0.2) (layer "B.Cu") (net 6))
 (segment (start 127.091 88.02395) (end 127.091 88.93605) (width 0.2) (layer "B.Cu") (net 6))
 (segment (start 125.99 92.459) (end 126.44605 92.459) (width 0.2) (layer "B.Cu") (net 6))
 (segment (start 124.478 97.9183) (end 124.478 104.3772) (width 0.2) (layer "B.Cu") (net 6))
 (segment (start 126.44605 87.379) (end 127.091 88.02395) (width 0.2) (layer "B.Cu") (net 6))
 (segment (start 125.99 106.9146) (end 126.9991 107.9237) (width 0.2) (layer "B.Cu") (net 6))
 (segment (start 136.4337 107.9237) (end 137.94 109.43) (width 0.2) (layer "B.Cu") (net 6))
 (segment (start 125.99 85.94) (end 125.99 87.379) (width 0.2) (layer "B.Cu") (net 6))
 (segment (start 125.99 92.121) (end 125.99 92.459) (width 0.2) (layer "B.Cu") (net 6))
 (segment (start 124.478 104.3772) (end 125.99 105.8892) (width 0.2) (layer "B.Cu") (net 6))
 (segment (start 125.53395 94.999) (end 124.889 95.64395) (width 0.2) (layer "B.Cu") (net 6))
 (segment (start 124.478 97.9183) (end 124.478 103.4048) (width 0.2) (layer "B.Cu") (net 6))
 (segment (start 126.44605 92.459) (end 127.091 93.10395) (width 0.2) (layer "B.Cu") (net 6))
 (segment (start 126.44605 92.121) (end 125.99 92.121) (width 0.2) (layer "B.Cu") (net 6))
 (segment (start 126.9991 107.9237) (end 136.4337 107.9237) (width 0.2) (layer "B.Cu") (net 6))
 (segment (start 127.091 91.47605) (end 126.44605 92.121) (width 0.2) (layer "B.Cu") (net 6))
 (segment (start 125.99 87.379) (end 126.44605 87.379) (width 0.2) (layer "B.Cu") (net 6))
 (segment (start 125.99 89.919) (end 126.44605 89.919) (width 0.2) (layer "B.Cu") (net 6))
 (segment (start 124.889 96.55605) (end 125.364625 97.031675) (width 0.2) (layer "B.Cu") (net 6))
 (segment (start 126.44605 94.661) (end 125.99 94.661) (width 0.2) (layer "B.Cu") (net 6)))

